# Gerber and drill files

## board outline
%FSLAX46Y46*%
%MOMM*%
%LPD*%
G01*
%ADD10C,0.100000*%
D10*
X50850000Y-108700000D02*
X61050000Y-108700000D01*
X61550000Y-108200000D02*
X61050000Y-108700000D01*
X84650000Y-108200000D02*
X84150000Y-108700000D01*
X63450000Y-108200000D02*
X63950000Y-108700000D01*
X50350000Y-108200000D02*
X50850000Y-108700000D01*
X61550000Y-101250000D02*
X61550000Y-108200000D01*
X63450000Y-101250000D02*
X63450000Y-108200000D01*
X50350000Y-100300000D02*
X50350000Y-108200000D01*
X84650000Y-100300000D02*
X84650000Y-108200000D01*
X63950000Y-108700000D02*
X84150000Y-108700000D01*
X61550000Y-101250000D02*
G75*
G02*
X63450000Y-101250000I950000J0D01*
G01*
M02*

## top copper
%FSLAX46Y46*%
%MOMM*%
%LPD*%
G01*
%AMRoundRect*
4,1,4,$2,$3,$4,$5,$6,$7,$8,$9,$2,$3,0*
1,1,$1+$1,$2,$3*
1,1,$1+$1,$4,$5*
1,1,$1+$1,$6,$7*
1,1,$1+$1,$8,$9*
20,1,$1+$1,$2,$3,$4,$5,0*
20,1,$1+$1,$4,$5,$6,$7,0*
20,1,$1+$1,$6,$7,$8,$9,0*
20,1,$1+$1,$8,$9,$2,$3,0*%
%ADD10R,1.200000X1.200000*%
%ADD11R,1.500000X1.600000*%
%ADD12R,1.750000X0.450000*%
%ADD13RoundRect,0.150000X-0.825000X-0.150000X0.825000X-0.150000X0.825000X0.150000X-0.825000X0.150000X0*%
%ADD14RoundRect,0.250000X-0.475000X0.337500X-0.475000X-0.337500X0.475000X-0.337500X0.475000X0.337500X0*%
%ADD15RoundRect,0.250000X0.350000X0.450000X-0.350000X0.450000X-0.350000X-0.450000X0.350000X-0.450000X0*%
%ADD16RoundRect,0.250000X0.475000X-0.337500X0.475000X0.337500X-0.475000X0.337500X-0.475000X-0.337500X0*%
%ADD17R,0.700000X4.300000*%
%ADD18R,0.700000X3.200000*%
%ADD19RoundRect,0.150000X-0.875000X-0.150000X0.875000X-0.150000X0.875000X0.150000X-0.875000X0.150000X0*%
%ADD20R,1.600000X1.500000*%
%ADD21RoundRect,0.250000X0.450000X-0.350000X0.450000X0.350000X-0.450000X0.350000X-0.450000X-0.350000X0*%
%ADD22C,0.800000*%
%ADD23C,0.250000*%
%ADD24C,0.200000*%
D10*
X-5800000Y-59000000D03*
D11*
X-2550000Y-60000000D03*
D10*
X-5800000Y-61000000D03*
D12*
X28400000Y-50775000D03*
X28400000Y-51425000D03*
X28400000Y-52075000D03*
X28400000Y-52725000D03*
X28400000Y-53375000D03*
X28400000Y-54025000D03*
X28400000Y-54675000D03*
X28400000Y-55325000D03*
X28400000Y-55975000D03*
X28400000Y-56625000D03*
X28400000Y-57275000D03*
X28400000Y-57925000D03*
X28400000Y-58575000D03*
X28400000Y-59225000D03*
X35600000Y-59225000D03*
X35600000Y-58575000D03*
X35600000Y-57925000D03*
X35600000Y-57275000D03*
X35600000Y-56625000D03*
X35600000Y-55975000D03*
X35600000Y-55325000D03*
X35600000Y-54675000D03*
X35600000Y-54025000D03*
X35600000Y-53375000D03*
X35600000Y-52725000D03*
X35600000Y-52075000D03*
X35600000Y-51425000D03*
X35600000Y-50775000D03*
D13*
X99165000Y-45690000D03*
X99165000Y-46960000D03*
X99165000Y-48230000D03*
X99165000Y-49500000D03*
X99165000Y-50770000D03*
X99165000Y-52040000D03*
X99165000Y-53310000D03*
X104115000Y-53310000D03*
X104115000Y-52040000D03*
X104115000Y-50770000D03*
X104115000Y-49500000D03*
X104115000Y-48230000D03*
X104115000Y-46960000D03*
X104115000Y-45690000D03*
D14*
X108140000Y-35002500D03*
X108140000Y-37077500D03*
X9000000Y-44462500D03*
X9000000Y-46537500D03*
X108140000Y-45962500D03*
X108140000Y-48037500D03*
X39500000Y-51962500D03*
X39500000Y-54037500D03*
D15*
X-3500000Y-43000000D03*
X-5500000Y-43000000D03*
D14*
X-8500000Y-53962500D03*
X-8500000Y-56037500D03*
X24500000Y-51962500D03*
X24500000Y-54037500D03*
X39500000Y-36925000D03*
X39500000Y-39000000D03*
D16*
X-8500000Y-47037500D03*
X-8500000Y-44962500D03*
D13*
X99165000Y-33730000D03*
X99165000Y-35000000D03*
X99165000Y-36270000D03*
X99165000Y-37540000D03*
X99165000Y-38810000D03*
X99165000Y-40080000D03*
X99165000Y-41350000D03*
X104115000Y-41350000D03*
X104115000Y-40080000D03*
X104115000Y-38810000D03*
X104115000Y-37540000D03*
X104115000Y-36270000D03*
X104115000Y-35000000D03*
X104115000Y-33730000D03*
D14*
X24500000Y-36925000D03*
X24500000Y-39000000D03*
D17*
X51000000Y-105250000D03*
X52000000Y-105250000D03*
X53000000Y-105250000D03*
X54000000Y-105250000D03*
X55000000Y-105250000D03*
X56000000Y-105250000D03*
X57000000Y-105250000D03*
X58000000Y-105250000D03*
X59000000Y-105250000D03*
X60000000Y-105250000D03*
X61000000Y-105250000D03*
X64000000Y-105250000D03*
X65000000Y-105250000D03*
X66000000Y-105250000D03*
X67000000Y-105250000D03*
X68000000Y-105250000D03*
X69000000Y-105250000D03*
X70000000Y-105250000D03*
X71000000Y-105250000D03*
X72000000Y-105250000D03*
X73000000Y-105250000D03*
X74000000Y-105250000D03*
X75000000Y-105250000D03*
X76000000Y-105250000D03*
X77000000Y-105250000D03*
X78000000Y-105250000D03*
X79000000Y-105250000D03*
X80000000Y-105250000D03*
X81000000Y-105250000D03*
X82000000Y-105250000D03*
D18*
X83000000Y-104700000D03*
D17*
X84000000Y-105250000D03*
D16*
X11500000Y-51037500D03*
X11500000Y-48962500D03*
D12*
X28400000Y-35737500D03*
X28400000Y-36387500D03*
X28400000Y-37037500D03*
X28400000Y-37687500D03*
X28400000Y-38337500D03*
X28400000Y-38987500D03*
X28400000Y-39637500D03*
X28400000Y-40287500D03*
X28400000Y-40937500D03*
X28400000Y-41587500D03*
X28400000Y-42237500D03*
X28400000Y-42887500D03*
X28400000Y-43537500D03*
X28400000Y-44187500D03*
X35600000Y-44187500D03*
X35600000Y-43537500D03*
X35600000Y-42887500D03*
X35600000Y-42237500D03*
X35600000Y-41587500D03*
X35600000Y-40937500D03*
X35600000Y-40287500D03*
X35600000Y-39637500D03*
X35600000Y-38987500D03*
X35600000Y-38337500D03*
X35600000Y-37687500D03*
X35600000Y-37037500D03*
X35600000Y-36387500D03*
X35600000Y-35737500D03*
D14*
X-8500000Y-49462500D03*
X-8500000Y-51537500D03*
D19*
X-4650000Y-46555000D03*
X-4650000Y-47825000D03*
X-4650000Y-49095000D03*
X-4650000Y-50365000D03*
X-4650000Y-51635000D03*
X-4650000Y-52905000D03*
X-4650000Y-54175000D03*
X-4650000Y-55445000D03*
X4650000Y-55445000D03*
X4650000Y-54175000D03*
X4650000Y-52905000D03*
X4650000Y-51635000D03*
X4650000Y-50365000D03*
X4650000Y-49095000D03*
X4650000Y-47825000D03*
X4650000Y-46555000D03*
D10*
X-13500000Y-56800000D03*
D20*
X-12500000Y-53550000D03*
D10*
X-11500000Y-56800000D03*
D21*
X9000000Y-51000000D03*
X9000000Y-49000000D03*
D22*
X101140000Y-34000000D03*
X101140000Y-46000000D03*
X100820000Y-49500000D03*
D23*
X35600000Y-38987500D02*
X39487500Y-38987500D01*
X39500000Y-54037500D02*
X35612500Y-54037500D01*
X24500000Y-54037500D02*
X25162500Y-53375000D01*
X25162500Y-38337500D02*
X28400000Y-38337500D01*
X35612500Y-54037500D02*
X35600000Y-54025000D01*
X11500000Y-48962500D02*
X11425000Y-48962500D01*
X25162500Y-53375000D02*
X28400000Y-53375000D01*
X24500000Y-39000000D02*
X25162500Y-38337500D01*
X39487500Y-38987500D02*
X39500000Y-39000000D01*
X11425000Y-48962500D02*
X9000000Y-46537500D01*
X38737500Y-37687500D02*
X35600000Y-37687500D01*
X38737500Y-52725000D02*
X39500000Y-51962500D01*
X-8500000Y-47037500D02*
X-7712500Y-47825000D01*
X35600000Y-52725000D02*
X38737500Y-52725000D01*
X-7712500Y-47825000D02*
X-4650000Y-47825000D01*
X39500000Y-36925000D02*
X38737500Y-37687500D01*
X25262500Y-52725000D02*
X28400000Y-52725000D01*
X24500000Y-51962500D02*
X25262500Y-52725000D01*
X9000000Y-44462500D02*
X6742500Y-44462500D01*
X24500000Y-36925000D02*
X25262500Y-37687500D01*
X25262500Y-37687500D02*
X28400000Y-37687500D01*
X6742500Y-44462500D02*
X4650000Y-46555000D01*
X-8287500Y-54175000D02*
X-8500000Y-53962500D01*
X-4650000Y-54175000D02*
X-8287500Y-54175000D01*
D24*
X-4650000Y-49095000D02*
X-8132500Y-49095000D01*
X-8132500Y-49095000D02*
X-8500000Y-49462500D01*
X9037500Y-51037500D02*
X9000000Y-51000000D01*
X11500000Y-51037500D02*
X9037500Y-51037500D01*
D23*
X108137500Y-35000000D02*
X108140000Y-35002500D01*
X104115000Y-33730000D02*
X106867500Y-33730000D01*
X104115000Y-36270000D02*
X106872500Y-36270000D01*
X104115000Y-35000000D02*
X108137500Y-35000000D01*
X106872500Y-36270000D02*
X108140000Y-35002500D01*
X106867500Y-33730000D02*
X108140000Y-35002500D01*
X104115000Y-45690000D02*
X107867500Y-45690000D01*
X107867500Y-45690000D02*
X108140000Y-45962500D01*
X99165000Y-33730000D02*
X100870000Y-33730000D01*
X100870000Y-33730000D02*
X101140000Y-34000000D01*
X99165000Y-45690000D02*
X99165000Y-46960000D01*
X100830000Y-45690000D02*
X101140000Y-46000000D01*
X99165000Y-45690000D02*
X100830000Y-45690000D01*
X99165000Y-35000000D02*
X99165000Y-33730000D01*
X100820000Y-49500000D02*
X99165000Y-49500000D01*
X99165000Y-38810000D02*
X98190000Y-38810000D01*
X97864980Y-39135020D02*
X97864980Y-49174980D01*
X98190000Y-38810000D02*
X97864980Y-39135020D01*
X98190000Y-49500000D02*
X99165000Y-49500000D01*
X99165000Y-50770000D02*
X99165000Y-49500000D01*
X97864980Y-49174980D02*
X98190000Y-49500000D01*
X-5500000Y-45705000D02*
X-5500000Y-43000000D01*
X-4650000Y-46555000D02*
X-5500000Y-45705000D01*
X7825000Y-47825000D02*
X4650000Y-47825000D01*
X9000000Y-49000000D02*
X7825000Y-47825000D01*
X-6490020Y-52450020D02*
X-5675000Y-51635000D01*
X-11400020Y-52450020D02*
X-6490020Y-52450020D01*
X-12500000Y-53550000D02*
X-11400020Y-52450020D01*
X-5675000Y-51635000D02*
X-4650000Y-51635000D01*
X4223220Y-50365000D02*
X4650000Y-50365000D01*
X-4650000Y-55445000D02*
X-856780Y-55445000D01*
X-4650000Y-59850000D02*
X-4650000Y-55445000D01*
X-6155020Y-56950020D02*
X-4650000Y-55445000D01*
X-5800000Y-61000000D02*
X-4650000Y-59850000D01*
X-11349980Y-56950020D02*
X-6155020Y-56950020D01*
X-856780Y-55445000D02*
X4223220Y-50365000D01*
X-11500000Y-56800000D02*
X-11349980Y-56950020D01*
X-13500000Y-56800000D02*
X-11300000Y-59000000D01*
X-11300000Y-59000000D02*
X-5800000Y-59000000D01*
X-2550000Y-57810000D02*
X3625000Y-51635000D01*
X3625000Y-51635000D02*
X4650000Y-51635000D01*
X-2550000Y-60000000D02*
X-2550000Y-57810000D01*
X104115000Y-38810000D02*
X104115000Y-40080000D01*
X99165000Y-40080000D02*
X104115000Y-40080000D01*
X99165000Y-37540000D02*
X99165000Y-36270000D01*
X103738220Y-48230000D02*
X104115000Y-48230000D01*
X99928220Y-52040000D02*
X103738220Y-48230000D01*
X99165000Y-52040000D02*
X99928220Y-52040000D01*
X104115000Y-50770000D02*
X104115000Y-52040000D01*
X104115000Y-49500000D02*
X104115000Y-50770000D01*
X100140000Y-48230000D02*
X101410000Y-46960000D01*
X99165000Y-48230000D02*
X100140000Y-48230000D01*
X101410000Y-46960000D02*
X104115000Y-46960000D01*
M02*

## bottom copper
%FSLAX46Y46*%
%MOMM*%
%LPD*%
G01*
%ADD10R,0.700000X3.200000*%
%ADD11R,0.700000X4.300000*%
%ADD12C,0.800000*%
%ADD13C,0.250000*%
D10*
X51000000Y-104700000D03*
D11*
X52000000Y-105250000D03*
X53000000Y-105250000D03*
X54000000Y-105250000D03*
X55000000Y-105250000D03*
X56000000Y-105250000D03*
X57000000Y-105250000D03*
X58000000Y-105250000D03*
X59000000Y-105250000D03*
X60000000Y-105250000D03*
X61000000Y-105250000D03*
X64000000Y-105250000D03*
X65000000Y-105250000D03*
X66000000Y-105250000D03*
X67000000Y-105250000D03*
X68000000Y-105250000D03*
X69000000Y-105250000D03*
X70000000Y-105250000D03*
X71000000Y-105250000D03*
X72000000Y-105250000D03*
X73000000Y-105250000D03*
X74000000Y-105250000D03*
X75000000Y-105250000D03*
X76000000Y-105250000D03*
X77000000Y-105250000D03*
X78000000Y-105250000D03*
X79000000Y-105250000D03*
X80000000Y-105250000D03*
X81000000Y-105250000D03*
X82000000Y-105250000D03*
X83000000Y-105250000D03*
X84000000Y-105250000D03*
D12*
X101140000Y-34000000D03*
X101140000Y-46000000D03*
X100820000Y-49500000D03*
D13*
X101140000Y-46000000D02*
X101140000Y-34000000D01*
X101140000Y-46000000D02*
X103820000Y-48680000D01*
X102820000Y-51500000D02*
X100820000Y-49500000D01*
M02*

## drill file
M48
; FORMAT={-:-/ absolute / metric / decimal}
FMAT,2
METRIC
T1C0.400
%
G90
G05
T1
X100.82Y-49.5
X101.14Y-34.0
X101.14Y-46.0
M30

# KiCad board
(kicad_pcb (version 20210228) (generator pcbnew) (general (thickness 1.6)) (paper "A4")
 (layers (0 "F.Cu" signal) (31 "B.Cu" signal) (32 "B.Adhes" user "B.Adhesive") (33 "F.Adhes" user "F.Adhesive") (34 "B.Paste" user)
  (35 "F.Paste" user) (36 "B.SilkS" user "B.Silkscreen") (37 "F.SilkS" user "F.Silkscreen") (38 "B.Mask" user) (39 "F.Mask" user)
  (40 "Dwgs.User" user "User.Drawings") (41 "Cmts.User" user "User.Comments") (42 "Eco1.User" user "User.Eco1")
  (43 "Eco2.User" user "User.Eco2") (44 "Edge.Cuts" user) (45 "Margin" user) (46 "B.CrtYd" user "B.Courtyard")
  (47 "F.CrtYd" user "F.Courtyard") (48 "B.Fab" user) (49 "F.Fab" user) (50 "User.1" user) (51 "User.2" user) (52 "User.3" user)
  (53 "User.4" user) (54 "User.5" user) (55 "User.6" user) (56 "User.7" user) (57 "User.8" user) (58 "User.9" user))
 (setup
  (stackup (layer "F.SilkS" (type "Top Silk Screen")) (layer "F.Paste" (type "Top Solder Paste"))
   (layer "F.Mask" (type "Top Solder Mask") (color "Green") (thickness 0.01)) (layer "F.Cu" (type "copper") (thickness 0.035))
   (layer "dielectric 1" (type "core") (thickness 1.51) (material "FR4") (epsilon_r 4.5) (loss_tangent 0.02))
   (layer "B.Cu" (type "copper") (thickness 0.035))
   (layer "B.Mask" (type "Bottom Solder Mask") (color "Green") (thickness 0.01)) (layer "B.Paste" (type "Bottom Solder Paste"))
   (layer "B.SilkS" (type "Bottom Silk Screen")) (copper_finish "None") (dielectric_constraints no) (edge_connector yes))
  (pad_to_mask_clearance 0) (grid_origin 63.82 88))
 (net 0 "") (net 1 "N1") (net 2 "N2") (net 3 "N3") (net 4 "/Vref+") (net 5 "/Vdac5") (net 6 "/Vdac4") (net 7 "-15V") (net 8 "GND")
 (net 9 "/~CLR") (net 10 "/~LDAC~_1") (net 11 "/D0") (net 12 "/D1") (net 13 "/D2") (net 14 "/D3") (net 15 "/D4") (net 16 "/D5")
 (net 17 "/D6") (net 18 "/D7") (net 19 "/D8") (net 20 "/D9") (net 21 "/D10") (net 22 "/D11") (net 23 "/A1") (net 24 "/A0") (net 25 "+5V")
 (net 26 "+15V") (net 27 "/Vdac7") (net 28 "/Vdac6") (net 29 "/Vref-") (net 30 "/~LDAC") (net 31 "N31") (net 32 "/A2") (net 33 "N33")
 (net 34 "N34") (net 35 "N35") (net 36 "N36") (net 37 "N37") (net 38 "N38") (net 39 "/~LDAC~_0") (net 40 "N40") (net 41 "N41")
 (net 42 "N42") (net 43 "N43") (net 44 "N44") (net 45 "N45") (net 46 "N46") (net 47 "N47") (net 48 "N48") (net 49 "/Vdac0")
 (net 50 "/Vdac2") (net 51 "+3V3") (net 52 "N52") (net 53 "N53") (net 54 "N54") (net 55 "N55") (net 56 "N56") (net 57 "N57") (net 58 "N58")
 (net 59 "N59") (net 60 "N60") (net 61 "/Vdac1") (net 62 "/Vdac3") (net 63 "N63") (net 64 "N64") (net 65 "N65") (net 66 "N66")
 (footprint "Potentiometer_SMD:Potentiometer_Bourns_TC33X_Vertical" (layer "F.Cu") (at -4 60)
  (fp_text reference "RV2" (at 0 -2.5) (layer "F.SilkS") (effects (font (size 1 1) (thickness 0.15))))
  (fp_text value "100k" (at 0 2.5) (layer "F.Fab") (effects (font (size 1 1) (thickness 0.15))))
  (pad "1" smd rect (at -1.8 -1) (locked) (size 1.2 1.2) (layers "F.Cu" "F.Paste" "F.Mask") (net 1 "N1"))
  (pad "2" smd rect (at 1.45 0) (locked) (size 1.5 1.6) (layers "F.Cu" "F.Paste" "F.Mask") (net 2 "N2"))
  (pad "3" smd rect (at -1.8 1) (locked) (size 1.2 1.2) (layers "F.Cu" "F.Paste" "F.Mask") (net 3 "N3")))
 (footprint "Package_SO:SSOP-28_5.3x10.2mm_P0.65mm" (layer "F.Cu") (at 32 55)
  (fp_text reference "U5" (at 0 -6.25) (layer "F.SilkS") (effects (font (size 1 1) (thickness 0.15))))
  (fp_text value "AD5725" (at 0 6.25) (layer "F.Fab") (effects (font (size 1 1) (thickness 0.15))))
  (pad "1" smd rect (at -3.6 -4.225) (locked) (size 1.75 0.45) (layers "F.Cu" "F.Paste" "F.Mask") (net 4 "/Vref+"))
  (pad "2" smd rect (at -3.6 -3.575) (locked) (size 1.75 0.45) (layers "F.Cu" "F.Paste" "F.Mask") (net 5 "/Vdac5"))
  (pad "3" smd rect (at -3.6 -2.925) (locked) (size 1.75 0.45) (layers "F.Cu" "F.Paste" "F.Mask") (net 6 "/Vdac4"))
  (pad "4" smd rect (at -3.6 -2.275) (locked) (size 1.75 0.45) (layers "F.Cu" "F.Paste" "F.Mask") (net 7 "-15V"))
  (pad "5" smd rect (at -3.6 -1.625) (locked) (size 1.75 0.45) (layers "F.Cu" "F.Paste" "F.Mask") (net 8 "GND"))
  (pad "6" smd rect (at -3.6 -0.975) (locked) (size 1.75 0.45) (layers "F.Cu" "F.Paste" "F.Mask") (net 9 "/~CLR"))
  (pad "7" smd rect (at -3.6 -0.325) (locked) (size 1.75 0.45) (layers "F.Cu" "F.Paste" "F.Mask") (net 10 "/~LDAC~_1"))
  (pad "8" smd rect (at -3.6 0.325) (locked) (size 1.75 0.45) (layers "F.Cu" "F.Paste" "F.Mask") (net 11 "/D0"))
  (pad "9" smd rect (at -3.6 0.975) (locked) (size 1.75 0.45) (layers "F.Cu" "F.Paste" "F.Mask") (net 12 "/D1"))
  (pad "10" smd rect (at -3.6 1.625) (locked) (size 1.75 0.45) (layers "F.Cu" "F.Paste" "F.Mask") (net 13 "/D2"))
  (pad "11" smd rect (at -3.6 2.275) (locked) (size 1.75 0.45) (layers "F.Cu" "F.Paste" "F.Mask") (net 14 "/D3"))
  (pad "12" smd rect (at -3.6 2.925) (locked) (size 1.75 0.45) (layers "F.Cu" "F.Paste" "F.Mask") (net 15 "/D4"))
  (pad "13" smd rect (at -3.6 3.575) (locked) (size 1.75 0.45) (layers "F.Cu" "F.Paste" "F.Mask") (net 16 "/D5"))
  (pad "14" smd rect (at -3.6 4.225) (locked) (size 1.75 0.45) (layers "F.Cu" "F.Paste" "F.Mask") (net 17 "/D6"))
  (pad "15" smd rect (at 3.6 4.225) (locked) (size 1.75 0.45) (layers "F.Cu" "F.Paste" "F.Mask") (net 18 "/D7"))
  (pad "16" smd rect (at 3.6 3.575) (locked) (size 1.75 0.45) (layers "F.Cu" "F.Paste" "F.Mask") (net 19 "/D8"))
  (pad "17" smd rect (at 3.6 2.925) (locked) (size 1.75 0.45) (layers "F.Cu" "F.Paste" "F.Mask") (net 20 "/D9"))
  (pad "18" smd rect (at 3.6 2.275) (locked) (size 1.75 0.45) (layers "F.Cu" "F.Paste" "F.Mask") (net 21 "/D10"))
  (pad "19" smd rect (at 3.6 1.625) (locked) (size 1.75 0.45) (layers "F.Cu" "F.Paste" "F.Mask") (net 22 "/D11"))
  (pad "20" smd rect (at 3.6 0.975) (locked) (size 1.75 0.45) (layers "F.Cu" "F.Paste" "F.Mask") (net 8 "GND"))
  (pad "21" smd rect (at 3.6 0.325) (locked) (size 1.75 0.45) (layers "F.Cu" "F.Paste" "F.Mask") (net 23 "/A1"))
  (pad "22" smd rect (at 3.6 -0.325) (locked) (size 1.75 0.45) (layers "F.Cu" "F.Paste" "F.Mask") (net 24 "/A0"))
  (pad "23" smd rect (at 3.6 -0.975) (locked) (size 1.75 0.45) (layers "F.Cu" "F.Paste" "F.Mask") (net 8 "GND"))
  (pad "24" smd rect (at 3.6 -1.625) (locked) (size 1.75 0.45) (layers "F.Cu" "F.Paste" "F.Mask") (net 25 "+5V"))
  (pad "25" smd rect (at 3.6 -2.275) (locked) (size 1.75 0.45) (layers "F.Cu" "F.Paste" "F.Mask") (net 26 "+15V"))
  (pad "26" smd rect (at 3.6 -2.925) (locked) (size 1.75 0.45) (layers "F.Cu" "F.Paste" "F.Mask") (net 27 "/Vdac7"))
  (pad "27" smd rect (at 3.6 -3.575) (locked) (size 1.75 0.45) (layers "F.Cu" "F.Paste" "F.Mask") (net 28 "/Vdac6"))
  (pad "28" smd rect (at 3.6 -4.225) (locked) (size 1.75 0.45) (layers "F.Cu" "F.Paste" "F.Mask") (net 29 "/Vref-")))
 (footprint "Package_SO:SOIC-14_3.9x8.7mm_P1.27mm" (layer "F.Cu") (at 101.64 49.5)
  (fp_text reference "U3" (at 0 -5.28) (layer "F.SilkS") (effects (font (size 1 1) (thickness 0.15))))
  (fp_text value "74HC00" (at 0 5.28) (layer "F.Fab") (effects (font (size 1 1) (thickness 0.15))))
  (pad "1" smd roundrect (at -2.475 -3.81) (locked) (size 1.95 0.6) (layers "F.Cu" "F.Paste" "F.Mask") (roundrect_rratio 0.25)
   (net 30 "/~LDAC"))
  (pad "2" smd roundrect (at -2.475 -2.54) (locked) (size 1.95 0.6) (layers "F.Cu" "F.Paste" "F.Mask") (roundrect_rratio 0.25)
   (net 30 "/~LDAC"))
  (pad "3" smd roundrect (at -2.475 -1.27) (locked) (size 1.95 0.6) (layers "F.Cu" "F.Paste" "F.Mask") (roundrect_rratio 0.25)
   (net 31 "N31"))
  (pad "4" smd roundrect (at -2.475 0) (locked) (size 1.95 0.6) (layers "F.Cu" "F.Paste" "F.Mask") (roundrect_rratio 0.25) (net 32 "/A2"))
  (pad "5" smd roundrect (at -2.475 1.27) (locked) (size 1.95 0.6) (layers "F.Cu" "F.Paste" "F.Mask") (roundrect_rratio 0.25) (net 32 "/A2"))
  (pad "6" smd roundrect (at -2.475 2.54) (locked) (size 1.95 0.6) (layers "F.Cu" "F.Paste" "F.Mask") (roundrect_rratio 0.25) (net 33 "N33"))
  (pad "7" smd roundrect (at -2.475 3.81) (locked) (size 1.95 0.6) (layers "F.Cu" "F.Paste" "F.Mask") (roundrect_rratio 0.25) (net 8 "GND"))
  (pad "8" smd roundrect (at 2.475 3.81) (locked) (size 1.95 0.6) (layers "F.Cu" "F.Paste" "F.Mask") (roundrect_rratio 0.25)
   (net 10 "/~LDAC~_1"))
  (pad "9" smd roundrect (at 2.475 2.54) (locked) (size 1.95 0.6) (layers "F.Cu" "F.Paste" "F.Mask") (roundrect_rratio 0.25) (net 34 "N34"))
  (pad "10" smd roundrect (at 2.475 1.27) (locked) (size 1.95 0.6) (layers "F.Cu" "F.Paste" "F.Mask") (roundrect_rratio 0.25) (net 34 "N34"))
  (pad "11" smd roundrect (at 2.475 0) (locked) (size 1.95 0.6) (layers "F.Cu" "F.Paste" "F.Mask") (roundrect_rratio 0.25) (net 34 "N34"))
  (pad "12" smd roundrect (at 2.475 -1.27) (locked) (size 1.95 0.6) (layers "F.Cu" "F.Paste" "F.Mask") (roundrect_rratio 0.25)
   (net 33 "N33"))
  (pad "13" smd roundrect (at 2.475 -2.54) (locked) (size 1.95 0.6) (layers "F.Cu" "F.Paste" "F.Mask") (roundrect_rratio 0.25)
   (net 31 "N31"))
  (pad "14" smd roundrect (at 2.475 -3.81) (locked) (size 1.95 0.6) (layers "F.Cu" "F.Paste" "F.Mask") (roundrect_rratio 0.25)
   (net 25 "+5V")))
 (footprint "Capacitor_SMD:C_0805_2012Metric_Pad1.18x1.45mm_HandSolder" (layer "F.Cu") (at 108.14 36.04 -90)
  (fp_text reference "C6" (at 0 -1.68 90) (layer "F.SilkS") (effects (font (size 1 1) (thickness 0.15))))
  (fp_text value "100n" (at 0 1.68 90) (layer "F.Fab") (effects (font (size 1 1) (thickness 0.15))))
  (pad "1" smd roundrect (at -1.0375 0 270) (locked) (size 1.175 1.45) (layers "F.Cu" "F.Paste" "F.Mask") (roundrect_rratio 0.212766)
   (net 25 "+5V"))
  (pad "2" smd roundrect (at 1.0375 0 270) (locked) (size 1.175 1.45) (layers "F.Cu" "F.Paste" "F.Mask") (roundrect_rratio 0.212766)
   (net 8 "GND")))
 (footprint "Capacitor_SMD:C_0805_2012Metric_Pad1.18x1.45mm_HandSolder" (layer "F.Cu") (at 9 45.5 -90)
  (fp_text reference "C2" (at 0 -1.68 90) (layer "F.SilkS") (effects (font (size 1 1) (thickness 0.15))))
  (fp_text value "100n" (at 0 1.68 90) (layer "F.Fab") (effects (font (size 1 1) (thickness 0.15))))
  (pad "1" smd roundrect (at -1.0375 0 270) (locked) (size 1.175 1.45) (layers "F.Cu" "F.Paste" "F.Mask") (roundrect_rratio 0.212766)
   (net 7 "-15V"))
  (pad "2" smd roundrect (at 1.0375 0 270) (locked) (size 1.175 1.45) (layers "F.Cu" "F.Paste" "F.Mask") (roundrect_rratio 0.212766)
   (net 8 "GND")))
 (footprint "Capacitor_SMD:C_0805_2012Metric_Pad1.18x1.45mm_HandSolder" (layer "F.Cu") (at 108.14 47 -90)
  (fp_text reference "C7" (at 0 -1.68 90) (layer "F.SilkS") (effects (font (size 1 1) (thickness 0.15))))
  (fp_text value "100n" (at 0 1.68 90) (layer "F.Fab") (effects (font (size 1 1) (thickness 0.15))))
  (pad "1" smd roundrect (at -1.0375 0 270) (locked) (size 1.175 1.45) (layers "F.Cu" "F.Paste" "F.Mask") (roundrect_rratio 0.212766)
   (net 25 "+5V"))
  (pad "2" smd roundrect (at 1.0375 0 270) (locked) (size 1.175 1.45) (layers "F.Cu" "F.Paste" "F.Mask") (roundrect_rratio 0.212766)
   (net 8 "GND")))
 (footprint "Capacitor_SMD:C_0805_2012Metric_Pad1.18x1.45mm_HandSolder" (layer "F.Cu") (at 39.5 53 -90)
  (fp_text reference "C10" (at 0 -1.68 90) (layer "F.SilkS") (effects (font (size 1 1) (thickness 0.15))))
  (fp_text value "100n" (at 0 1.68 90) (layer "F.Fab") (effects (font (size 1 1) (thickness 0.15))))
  (pad "1" smd roundrect (at -1.0375 0 270) (locked) (size 1.175 1.45) (layers "F.Cu" "F.Paste" "F.Mask") (roundrect_rratio 0.212766)
   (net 26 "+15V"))
  (pad "2" smd roundrect (at 1.0375 0 270) (locked) (size 1.175 1.45) (layers "F.Cu" "F.Paste" "F.Mask") (roundrect_rratio 0.212766)
   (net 8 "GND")))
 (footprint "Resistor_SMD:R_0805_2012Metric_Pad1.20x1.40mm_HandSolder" (layer "F.Cu") (at -4.5 43 180)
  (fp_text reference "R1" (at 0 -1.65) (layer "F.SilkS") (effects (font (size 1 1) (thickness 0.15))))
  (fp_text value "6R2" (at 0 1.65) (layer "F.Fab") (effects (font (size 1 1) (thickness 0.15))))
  (pad "1" smd roundrect (at -1 0 180) (locked) (size 1.2 1.4) (layers "F.Cu" "F.Paste" "F.Mask") (roundrect_rratio 0.208333)
   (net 4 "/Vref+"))
  (pad "2" smd roundrect (at 1 0 180) (locked) (size 1.2 1.4) (layers "F.Cu" "F.Paste" "F.Mask") (roundrect_rratio 0.208333) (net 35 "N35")))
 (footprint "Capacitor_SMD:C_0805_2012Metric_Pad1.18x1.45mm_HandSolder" (layer "F.Cu") (at -8.5 55 -90)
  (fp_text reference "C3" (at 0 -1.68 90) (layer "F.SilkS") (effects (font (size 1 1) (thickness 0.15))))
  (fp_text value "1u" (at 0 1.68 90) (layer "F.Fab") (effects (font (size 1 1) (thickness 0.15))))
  (pad "1" smd roundrect (at -1.0375 0 270) (locked) (size 1.175 1.45) (layers "F.Cu" "F.Paste" "F.Mask") (roundrect_rratio 0.212766)
   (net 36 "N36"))
  (pad "2" smd roundrect (at 1.0375 0 270) (locked) (size 1.175 1.45) (layers "F.Cu" "F.Paste" "F.Mask") (roundrect_rratio 0.212766)
   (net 8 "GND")))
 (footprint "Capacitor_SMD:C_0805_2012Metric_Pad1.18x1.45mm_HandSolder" (layer "F.Cu") (at 24.5 53 -90)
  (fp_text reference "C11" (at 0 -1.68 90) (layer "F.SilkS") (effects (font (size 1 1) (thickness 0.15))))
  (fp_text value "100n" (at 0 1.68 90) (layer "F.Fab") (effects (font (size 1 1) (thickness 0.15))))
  (pad "1" smd roundrect (at -1.0375 0 270) (locked) (size 1.175 1.45) (layers "F.Cu" "F.Paste" "F.Mask") (roundrect_rratio 0.212766)
   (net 7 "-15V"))
  (pad "2" smd roundrect (at 1.0375 0 270) (locked) (size 1.175 1.45) (layers "F.Cu" "F.Paste" "F.Mask") (roundrect_rratio 0.212766)
   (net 8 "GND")))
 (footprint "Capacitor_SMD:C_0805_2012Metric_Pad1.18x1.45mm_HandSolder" (layer "F.Cu") (at 39.5 37.9625 -90)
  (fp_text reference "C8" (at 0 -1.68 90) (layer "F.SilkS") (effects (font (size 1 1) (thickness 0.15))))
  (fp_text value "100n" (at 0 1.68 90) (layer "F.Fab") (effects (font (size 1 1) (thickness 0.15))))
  (pad "1" smd roundrect (at -1.0375 0 270) (locked) (size 1.175 1.45) (layers "F.Cu" "F.Paste" "F.Mask") (roundrect_rratio 0.212766)
   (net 26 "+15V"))
  (pad "2" smd roundrect (at 1.0375 0 270) (locked) (size 1.175 1.45) (layers "F.Cu" "F.Paste" "F.Mask") (roundrect_rratio 0.212766)
   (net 8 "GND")))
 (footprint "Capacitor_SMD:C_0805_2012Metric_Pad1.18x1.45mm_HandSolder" (layer "F.Cu") (at -8.5 46 90)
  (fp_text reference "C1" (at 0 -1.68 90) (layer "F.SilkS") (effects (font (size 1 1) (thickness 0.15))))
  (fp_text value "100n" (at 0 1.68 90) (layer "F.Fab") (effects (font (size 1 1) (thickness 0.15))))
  (pad "1" smd roundrect (at -1.0375 0 90) (locked) (size 1.175 1.45) (layers "F.Cu" "F.Paste" "F.Mask") (roundrect_rratio 0.212766)
   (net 26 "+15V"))
  (pad "2" smd roundrect (at 1.0375 0 90) (locked) (size 1.175 1.45) (layers "F.Cu" "F.Paste" "F.Mask") (roundrect_rratio 0.212766)
   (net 8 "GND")))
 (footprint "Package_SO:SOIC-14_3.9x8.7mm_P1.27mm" (layer "F.Cu") (at 101.64 37.54)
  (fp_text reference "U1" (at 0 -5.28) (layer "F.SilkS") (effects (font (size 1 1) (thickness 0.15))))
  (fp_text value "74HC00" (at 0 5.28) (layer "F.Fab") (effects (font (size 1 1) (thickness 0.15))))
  (pad "1" smd roundrect (at -2.475 -3.81) (locked) (size 1.95 0.6) (layers "F.Cu" "F.Paste" "F.Mask") (roundrect_rratio 0.25)
   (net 30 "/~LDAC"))
  (pad "2" smd roundrect (at -2.475 -2.54) (locked) (size 1.95 0.6) (layers "F.Cu" "F.Paste" "F.Mask") (roundrect_rratio 0.25)
   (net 30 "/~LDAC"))
  (pad "3" smd roundrect (at -2.475 -1.27) (locked) (size 1.95 0.6) (layers "F.Cu" "F.Paste" "F.Mask") (roundrect_rratio 0.25)
   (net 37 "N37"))
  (pad "4" smd roundrect (at -2.475 0) (locked) (size 1.95 0.6) (layers "F.Cu" "F.Paste" "F.Mask") (roundrect_rratio 0.25) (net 37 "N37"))
  (pad "5" smd roundrect (at -2.475 1.27) (locked) (size 1.95 0.6) (layers "F.Cu" "F.Paste" "F.Mask") (roundrect_rratio 0.25) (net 32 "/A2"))
  (pad "6" smd roundrect (at -2.475 2.54) (locked) (size 1.95 0.6) (layers "F.Cu" "F.Paste" "F.Mask") (roundrect_rratio 0.25) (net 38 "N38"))
  (pad "7" smd roundrect (at -2.475 3.81) (locked) (size 1.95 0.6) (layers "F.Cu" "F.Paste" "F.Mask") (roundrect_rratio 0.25) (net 8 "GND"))
  (pad "8" smd roundrect (at 2.475 3.81) (locked) (size 1.95 0.6) (layers "F.Cu" "F.Paste" "F.Mask") (roundrect_rratio 0.25)
   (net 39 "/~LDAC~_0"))
  (pad "9" smd roundrect (at 2.475 2.54) (locked) (size 1.95 0.6) (layers "F.Cu" "F.Paste" "F.Mask") (roundrect_rratio 0.25) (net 38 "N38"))
  (pad "10" smd roundrect (at 2.475 1.27) (locked) (size 1.95 0.6) (layers "F.Cu" "F.Paste" "F.Mask") (roundrect_rratio 0.25) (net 38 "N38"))
  (pad "11" smd roundrect (at 2.475 0) (locked) (size 1.95 0.6) (layers "F.Cu" "F.Paste" "F.Mask") (roundrect_rratio 0.25) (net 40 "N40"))
  (pad "12" smd roundrect (at 2.475 -1.27) (locked) (size 1.95 0.6) (layers "F.Cu" "F.Paste" "F.Mask") (roundrect_rratio 0.25)
   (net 25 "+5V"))
  (pad "13" smd roundrect (at 2.475 -2.54) (locked) (size 1.95 0.6) (layers "F.Cu" "F.Paste" "F.Mask") (roundrect_rratio 0.25)
   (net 25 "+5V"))
  (pad "14" smd roundrect (at 2.475 -3.81) (locked) (size 1.95 0.6) (layers "F.Cu" "F.Paste" "F.Mask") (roundrect_rratio 0.25)
   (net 25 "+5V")))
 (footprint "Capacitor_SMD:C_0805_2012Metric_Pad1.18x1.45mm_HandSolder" (layer "F.Cu") (at 24.5 37.9625 -90)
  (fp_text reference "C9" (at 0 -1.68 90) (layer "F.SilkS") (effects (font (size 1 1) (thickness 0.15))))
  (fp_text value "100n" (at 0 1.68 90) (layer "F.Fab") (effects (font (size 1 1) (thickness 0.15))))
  (pad "1" smd roundrect (at -1.0375 0 270) (locked) (size 1.175 1.45) (layers "F.Cu" "F.Paste" "F.Mask") (roundrect_rratio 0.212766)
   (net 7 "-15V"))
  (pad "2" smd roundrect (at 1.0375 0 270) (locked) (size 1.175 1.45) (layers "F.Cu" "F.Paste" "F.Mask") (roundrect_rratio 0.212766)
   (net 8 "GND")))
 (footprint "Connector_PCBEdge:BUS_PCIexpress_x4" (layer "F.Cu") (at 51 105.25)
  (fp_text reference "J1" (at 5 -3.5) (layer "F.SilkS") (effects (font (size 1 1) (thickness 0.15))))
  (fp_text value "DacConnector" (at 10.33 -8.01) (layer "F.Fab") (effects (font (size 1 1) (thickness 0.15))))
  (fp_line (start -0.15 3.45) (end 10.05 3.45) (layer "Edge.Cuts") (width 0.1))
  (fp_line (start 10.55 2.95) (end 10.05 3.45) (layer "Edge.Cuts") (width 0.1))
  (fp_line (start 33.65 2.95) (end 33.15 3.45) (layer "Edge.Cuts") (width 0.1))
  (fp_line (start 12.45 2.95) (end 12.95 3.45) (layer "Edge.Cuts") (width 0.1))
  (fp_line (start -0.65 2.95) (end -0.15 3.45) (layer "Edge.Cuts") (width 0.1))
  (fp_line (start 10.55 -4) (end 10.55 2.95) (layer "Edge.Cuts") (width 0.1))
  (fp_line (start 12.45 -4) (end 12.45 2.95) (layer "Edge.Cuts") (width 0.1))
  (fp_line (start -0.65 -4.95) (end -0.65 2.95) (layer "Edge.Cuts") (width 0.1))
  (fp_line (start 33.65 -4.95) (end 33.65 2.95) (layer "Edge.Cuts") (width 0.1))
  (fp_line (start 12.95 3.45) (end 33.15 3.45) (layer "Edge.Cuts") (width 0.1))
  (fp_arc (start 11.5 -4) (end 12.45 -4) (angle -180) (layer "Edge.Cuts") (width 0.1))
  (pad "A1" connect rect (at 0 -0.55) (locked) (size 0.7 3.2) (layers "B.Cu" "B.Mask") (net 26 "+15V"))
  (pad "A2" connect rect (at 1 0) (locked) (size 0.7 4.3) (layers "B.Cu" "B.Mask") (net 8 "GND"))
  (pad "A3" connect rect (at 2 0) (locked) (size 0.7 4.3) (layers "B.Cu" "B.Mask") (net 7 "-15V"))
  (pad "A4" connect rect (at 3 0) (locked) (size 0.7 4.3) (layers "B.Cu" "B.Mask") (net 8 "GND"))
  (pad "A5" connect rect (at 4 0) (locked) (size 0.7 4.3) (layers "B.Cu" "B.Mask") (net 25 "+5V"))
  (pad "A6" connect rect (at 5 0) (locked) (size 0.7 4.3) (layers "B.Cu" "B.Mask") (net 11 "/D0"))
  (pad "A7" connect rect (at 6 0) (locked) (size 0.7 4.3) (layers "B.Cu" "B.Mask") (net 13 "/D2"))
  (pad "A8" connect rect (at 7 0) (locked) (size 0.7 4.3) (layers "B.Cu" "B.Mask") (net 15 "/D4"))
  (pad "A9" connect rect (at 8 0) (locked) (size 0.7 4.3) (layers "B.Cu" "B.Mask") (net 17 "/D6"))
  (pad "A10" connect rect (at 9 0) (locked) (size 0.7 4.3) (layers "B.Cu" "B.Mask") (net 19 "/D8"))
  (pad "A11" connect rect (at 10 0) (locked) (size 0.7 4.3) (layers "B.Cu" "B.Mask") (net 21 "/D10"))
  (pad "A12" connect rect (at 13 0) (locked) (size 0.7 4.3) (layers "B.Cu" "B.Mask") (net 24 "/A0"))
  (pad "A13" connect rect (at 14 0) (locked) (size 0.7 4.3) (layers "B.Cu" "B.Mask") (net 32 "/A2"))
  (pad "A14" connect rect (at 15 0) (locked) (size 0.7 4.3) (layers "B.Cu" "B.Mask") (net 30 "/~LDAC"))
  (pad "A15" connect rect (at 16 0) (locked) (size 0.7 4.3) (layers "B.Cu" "B.Mask") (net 8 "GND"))
  (pad "A16" connect rect (at 17 0) (locked) (size 0.7 4.3) (layers "B.Cu" "B.Mask") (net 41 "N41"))
  (pad "A17" connect rect (at 18 0) (locked) (size 0.7 4.3) (layers "B.Cu" "B.Mask") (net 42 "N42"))
  (pad "A18" connect rect (at 19 0) (locked) (size 0.7 4.3) (layers "B.Cu" "B.Mask") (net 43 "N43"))
  (pad "A19" connect rect (at 20 0) (locked) (size 0.7 4.3) (layers "B.Cu" "B.Mask") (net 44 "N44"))
  (pad "A20" connect rect (at 21 0) (locked) (size 0.7 4.3) (layers "B.Cu" "B.Mask") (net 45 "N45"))
  (pad "A21" connect rect (at 22 0) (locked) (size 0.7 4.3) (layers "B.Cu" "B.Mask") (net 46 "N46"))
  (pad "A22" connect rect (at 23 0) (locked) (size 0.7 4.3) (layers "B.Cu" "B.Mask") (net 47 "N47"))
  (pad "A23" connect rect (at 24 0) (locked) (size 0.7 4.3) (layers "B.Cu" "B.Mask") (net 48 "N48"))
  (pad "A24" connect rect (at 25 0) (locked) (size 0.7 4.3) (layers "B.Cu" "B.Mask") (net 8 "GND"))
  (pad "A25" connect rect (at 26 0) (locked) (size 0.7 4.3) (layers "B.Cu" "B.Mask") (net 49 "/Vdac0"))
  (pad "A26" connect rect (at 27 0) (locked) (size 0.7 4.3) (layers "B.Cu" "B.Mask") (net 8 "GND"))
  (pad "A27" connect rect (at 28 0) (locked) (size 0.7 4.3) (layers "B.Cu" "B.Mask") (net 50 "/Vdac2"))
  (pad "A28" connect rect (at 29 0) (locked) (size 0.7 4.3) (layers "B.Cu" "B.Mask") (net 8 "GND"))
  (pad "A29" connect rect (at 30 0) (locked) (size 0.7 4.3) (layers "B.Cu" "B.Mask") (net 6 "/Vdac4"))
  (pad "A30" connect rect (at 31 0) (locked) (size 0.7 4.3) (layers "B.Cu" "B.Mask") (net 8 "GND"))
  (pad "A31" connect rect (at 32 0) (locked) (size 0.7 4.3) (layers "B.Cu" "B.Mask") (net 28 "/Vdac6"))
  (pad "A32" connect rect (at 33 0) (locked) (size 0.7 4.3) (layers "B.Cu" "B.Mask") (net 8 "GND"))
  (pad "B1" connect rect (at 0 0) (locked) (size 0.7 4.3) (layers "F.Cu" "F.Mask") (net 26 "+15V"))
  (pad "B2" connect rect (at 1 0) (locked) (size 0.7 4.3) (layers "F.Cu" "F.Mask") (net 8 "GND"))
  (pad "B3" connect rect (at 2 0) (locked) (size 0.7 4.3) (layers "F.Cu" "F.Mask") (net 7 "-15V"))
  (pad "B4" connect rect (at 3 0) (locked) (size 0.7 4.3) (layers "F.Cu" "F.Mask") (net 8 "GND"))
  (pad "B5" connect rect (at 4 0) (locked) (size 0.7 4.3) (layers "F.Cu" "F.Mask") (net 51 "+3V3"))
  (pad "B6" connect rect (at 5 0) (locked) (size 0.7 4.3) (layers "F.Cu" "F.Mask") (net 12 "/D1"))
  (pad "B7" connect rect (at 6 0) (locked) (size 0.7 4.3) (layers "F.Cu" "F.Mask") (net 14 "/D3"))
  (pad "B8" connect rect (at 7 0) (locked) (size 0.7 4.3) (layers "F.Cu" "F.Mask") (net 16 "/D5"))
  (pad "B9" connect rect (at 8 0) (locked) (size 0.7 4.3) (layers "F.Cu" "F.Mask") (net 18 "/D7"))
  (pad "B10" connect rect (at 9 0) (locked) (size 0.7 4.3) (layers "F.Cu" "F.Mask") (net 20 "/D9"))
  (pad "B11" connect rect (at 10 0) (locked) (size 0.7 4.3) (layers "F.Cu" "F.Mask") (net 22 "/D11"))
  (pad "B12" connect rect (at 13 0) (locked) (size 0.7 4.3) (layers "F.Cu" "F.Mask") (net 23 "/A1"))
  (pad "B13" connect rect (at 14 0) (locked) (size 0.7 4.3) (layers "F.Cu" "F.Mask") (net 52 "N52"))
  (pad "B14" connect rect (at 15 0) (locked) (size 0.7 4.3) (layers "F.Cu" "F.Mask") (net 9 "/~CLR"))
  (pad "B15" connect rect (at 16 0) (locked) (size 0.7 4.3) (layers "F.Cu" "F.Mask") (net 8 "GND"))
  (pad "B16" connect rect (at 17 0) (locked) (size 0.7 4.3) (layers "F.Cu" "F.Mask") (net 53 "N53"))
  (pad "B17" connect rect (at 18 0) (locked) (size 0.7 4.3) (layers "F.Cu" "F.Mask") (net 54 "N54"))
  (pad "B18" connect rect (at 19 0) (locked) (size 0.7 4.3) (layers "F.Cu" "F.Mask") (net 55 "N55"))
  (pad "B19" connect rect (at 20 0) (locked) (size 0.7 4.3) (layers "F.Cu" "F.Mask") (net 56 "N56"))
  (pad "B20" connect rect (at 21 0) (locked) (size 0.7 4.3) (layers "F.Cu" "F.Mask") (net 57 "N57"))
  (pad "B21" connect rect (at 22 0) (locked) (size 0.7 4.3) (layers "F.Cu" "F.Mask") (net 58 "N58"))
  (pad "B22" connect rect (at 23 0) (locked) (size 0.7 4.3) (layers "F.Cu" "F.Mask") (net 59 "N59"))
  (pad "B23" connect rect (at 24 0) (locked) (size 0.7 4.3) (layers "F.Cu" "F.Mask") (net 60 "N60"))
  (pad "B24" connect rect (at 25 0) (locked) (size 0.7 4.3) (layers "F.Cu" "F.Mask") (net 8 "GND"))
  (pad "B25" connect rect (at 26 0) (locked) (size 0.7 4.3) (layers "F.Cu" "F.Mask") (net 8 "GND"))
  (pad "B26" connect rect (at 27 0) (locked) (size 0.7 4.3) (layers "F.Cu" "F.Mask") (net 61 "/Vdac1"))
  (pad "B27" connect rect (at 28 0) (locked) (size 0.7 4.3) (layers "F.Cu" "F.Mask") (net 8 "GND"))
  (pad "B28" connect rect (at 29 0) (locked) (size 0.7 4.3) (layers "F.Cu" "F.Mask") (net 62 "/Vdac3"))
  (pad "B29" connect rect (at 30 0) (locked) (size 0.7 4.3) (layers "F.Cu" "F.Mask") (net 8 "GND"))
  (pad "B30" connect rect (at 31 0) (locked) (size 0.7 4.3) (layers "F.Cu" "F.Mask") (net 5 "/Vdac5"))
  (pad "B31" connect rect (at 32 -0.55) (locked) (size 0.7 3.2) (layers "F.Cu" "F.Mask") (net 8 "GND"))
  (pad "B32" connect rect (at 33 0) (locked) (size 0.7 4.3) (layers "F.Cu" "F.Mask") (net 27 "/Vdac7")))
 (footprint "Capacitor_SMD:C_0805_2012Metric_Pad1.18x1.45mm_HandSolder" (layer "F.Cu") (at 11.5 50 90)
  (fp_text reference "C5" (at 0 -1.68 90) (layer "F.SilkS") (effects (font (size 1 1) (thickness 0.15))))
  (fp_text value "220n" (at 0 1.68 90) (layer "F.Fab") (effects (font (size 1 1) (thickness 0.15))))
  (pad "1" smd roundrect (at -1.0375 0 90) (locked) (size 1.175 1.45) (layers "F.Cu" "F.Paste" "F.Mask") (roundrect_rratio 0.212766)
   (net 29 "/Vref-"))
  (pad "2" smd roundrect (at 1.0375 0 90) (locked) (size 1.175 1.45) (layers "F.Cu" "F.Paste" "F.Mask") (roundrect_rratio 0.212766)
   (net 8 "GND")))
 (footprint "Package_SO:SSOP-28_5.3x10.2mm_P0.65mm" (layer "F.Cu") (at 32 39.9625)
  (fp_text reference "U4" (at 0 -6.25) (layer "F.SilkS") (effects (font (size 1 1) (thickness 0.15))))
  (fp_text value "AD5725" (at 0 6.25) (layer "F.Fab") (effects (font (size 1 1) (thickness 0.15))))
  (pad "1" smd rect (at -3.6 -4.225) (locked) (size 1.75 0.45) (layers "F.Cu" "F.Paste" "F.Mask") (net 4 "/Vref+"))
  (pad "2" smd rect (at -3.6 -3.575) (locked) (size 1.75 0.45) (layers "F.Cu" "F.Paste" "F.Mask") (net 61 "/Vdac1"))
  (pad "3" smd rect (at -3.6 -2.925) (locked) (size 1.75 0.45) (layers "F.Cu" "F.Paste" "F.Mask") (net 49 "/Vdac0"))
  (pad "4" smd rect (at -3.6 -2.275) (locked) (size 1.75 0.45) (layers "F.Cu" "F.Paste" "F.Mask") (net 7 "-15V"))
  (pad "5" smd rect (at -3.6 -1.625) (locked) (size 1.75 0.45) (layers "F.Cu" "F.Paste" "F.Mask") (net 8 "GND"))
  (pad "6" smd rect (at -3.6 -0.975) (locked) (size 1.75 0.45) (layers "F.Cu" "F.Paste" "F.Mask") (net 9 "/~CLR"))
  (pad "7" smd rect (at -3.6 -0.325) (locked) (size 1.75 0.45) (layers "F.Cu" "F.Paste" "F.Mask") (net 39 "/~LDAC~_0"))
  (pad "8" smd rect (at -3.6 0.325) (locked) (size 1.75 0.45) (layers "F.Cu" "F.Paste" "F.Mask") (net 11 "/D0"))
  (pad "9" smd rect (at -3.6 0.975) (locked) (size 1.75 0.45) (layers "F.Cu" "F.Paste" "F.Mask") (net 12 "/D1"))
  (pad "10" smd rect (at -3.6 1.625) (locked) (size 1.75 0.45) (layers "F.Cu" "F.Paste" "F.Mask") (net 13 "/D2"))
  (pad "11" smd rect (at -3.6 2.275) (locked) (size 1.75 0.45) (layers "F.Cu" "F.Paste" "F.Mask") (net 14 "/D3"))
  (pad "12" smd rect (at -3.6 2.925) (locked) (size 1.75 0.45) (layers "F.Cu" "F.Paste" "F.Mask") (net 15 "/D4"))
  (pad "13" smd rect (at -3.6 3.575) (locked) (size 1.75 0.45) (layers "F.Cu" "F.Paste" "F.Mask") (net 16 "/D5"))
  (pad "14" smd rect (at -3.6 4.225) (locked) (size 1.75 0.45) (layers "F.Cu" "F.Paste" "F.Mask") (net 17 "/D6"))
  (pad "15" smd rect (at 3.6 4.225) (locked) (size 1.75 0.45) (layers "F.Cu" "F.Paste" "F.Mask") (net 18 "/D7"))
  (pad "16" smd rect (at 3.6 3.575) (locked) (size 1.75 0.45) (layers "F.Cu" "F.Paste" "F.Mask") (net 19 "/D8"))
  (pad "17" smd rect (at 3.6 2.925) (locked) (size 1.75 0.45) (layers "F.Cu" "F.Paste" "F.Mask") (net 20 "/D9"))
  (pad "18" smd rect (at 3.6 2.275) (locked) (size 1.75 0.45) (layers "F.Cu" "F.Paste" "F.Mask") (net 21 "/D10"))
  (pad "19" smd rect (at 3.6 1.625) (locked) (size 1.75 0.45) (layers "F.Cu" "F.Paste" "F.Mask") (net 22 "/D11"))
  (pad "20" smd rect (at 3.6 0.975) (locked) (size 1.75 0.45) (layers "F.Cu" "F.Paste" "F.Mask") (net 8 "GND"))
  (pad "21" smd rect (at 3.6 0.325) (locked) (size 1.75 0.45) (layers "F.Cu" "F.Paste" "F.Mask") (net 23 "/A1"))
  (pad "22" smd rect (at 3.6 -0.325) (locked) (size 1.75 0.45) (layers "F.Cu" "F.Paste" "F.Mask") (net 24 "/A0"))
  (pad "23" smd rect (at 3.6 -0.975) (locked) (size 1.75 0.45) (layers "F.Cu" "F.Paste" "F.Mask") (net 8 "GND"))
  (pad "24" smd rect (at 3.6 -1.625) (locked) (size 1.75 0.45) (layers "F.Cu" "F.Paste" "F.Mask") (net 25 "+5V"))
  (pad "25" smd rect (at 3.6 -2.275) (locked) (size 1.75 0.45) (layers "F.Cu" "F.Paste" "F.Mask") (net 26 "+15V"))
  (pad "26" smd rect (at 3.6 -2.925) (locked) (size 1.75 0.45) (layers "F.Cu" "F.Paste" "F.Mask") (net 62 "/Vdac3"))
  (pad "27" smd rect (at 3.6 -3.575) (locked) (size 1.75 0.45) (layers "F.Cu" "F.Paste" "F.Mask") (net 50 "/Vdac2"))
  (pad "28" smd rect (at 3.6 -4.225) (locked) (size 1.75 0.45) (layers "F.Cu" "F.Paste" "F.Mask") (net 29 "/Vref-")))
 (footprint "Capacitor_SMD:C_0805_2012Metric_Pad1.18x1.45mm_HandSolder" (layer "F.Cu") (at -8.5 50.5 -90)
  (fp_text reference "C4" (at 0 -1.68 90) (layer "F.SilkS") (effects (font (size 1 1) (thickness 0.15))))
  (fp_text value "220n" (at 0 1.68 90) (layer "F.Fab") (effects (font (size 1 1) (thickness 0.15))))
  (pad "1" smd roundrect (at -1.0375 0 270) (locked) (size 1.175 1.45) (layers "F.Cu" "F.Paste" "F.Mask") (roundrect_rratio 0.212766)
   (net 4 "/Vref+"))
  (pad "2" smd roundrect (at 1.0375 0 270) (locked) (size 1.175 1.45) (layers "F.Cu" "F.Paste" "F.Mask") (roundrect_rratio 0.212766)
   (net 8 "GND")))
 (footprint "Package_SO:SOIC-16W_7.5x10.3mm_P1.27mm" (layer "F.Cu") (at 0 51)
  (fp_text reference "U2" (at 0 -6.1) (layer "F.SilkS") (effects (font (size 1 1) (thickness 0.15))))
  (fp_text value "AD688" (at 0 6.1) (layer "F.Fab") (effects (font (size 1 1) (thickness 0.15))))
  (pad "1" smd roundrect (at -4.65 -4.445) (locked) (size 2.05 0.6) (layers "F.Cu" "F.Paste" "F.Mask") (roundrect_rratio 0.25)
   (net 35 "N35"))
  (pad "2" smd roundrect (at -4.65 -3.175) (locked) (size 2.05 0.6) (layers "F.Cu" "F.Paste" "F.Mask") (roundrect_rratio 0.25)
   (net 26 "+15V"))
  (pad "3" smd roundrect (at -4.65 -1.905) (locked) (size 2.05 0.6) (layers "F.Cu" "F.Paste" "F.Mask") (roundrect_rratio 0.25)
   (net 4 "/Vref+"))
  (pad "4" smd roundrect (at -4.65 -0.635) (locked) (size 2.05 0.6) (layers "F.Cu" "F.Paste" "F.Mask") (roundrect_rratio 0.25) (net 1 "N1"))
  (pad "5" smd roundrect (at -4.65 0.635) (locked) (size 2.05 0.6) (layers "F.Cu" "F.Paste" "F.Mask") (roundrect_rratio 0.25) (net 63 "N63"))
  (pad "6" smd roundrect (at -4.65 1.905) (locked) (size 2.05 0.6) (layers "F.Cu" "F.Paste" "F.Mask") (roundrect_rratio 0.25) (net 1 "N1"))
  (pad "7" smd roundrect (at -4.65 3.175) (locked) (size 2.05 0.6) (layers "F.Cu" "F.Paste" "F.Mask") (roundrect_rratio 0.25) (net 36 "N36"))
  (pad "8" smd roundrect (at -4.65 4.445) (locked) (size 2.05 0.6) (layers "F.Cu" "F.Paste" "F.Mask") (roundrect_rratio 0.25) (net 3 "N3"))
  (pad "9" smd roundrect (at 4.65 4.445) (locked) (size 2.05 0.6) (layers "F.Cu" "F.Paste" "F.Mask") (roundrect_rratio 0.25) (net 8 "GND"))
  (pad "10" smd roundrect (at 4.65 3.175) (locked) (size 2.05 0.6) (layers "F.Cu" "F.Paste" "F.Mask") (roundrect_rratio 0.25) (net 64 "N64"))
  (pad "11" smd roundrect (at 4.65 1.905) (locked) (size 2.05 0.6) (layers "F.Cu" "F.Paste" "F.Mask") (roundrect_rratio 0.25) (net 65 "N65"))
  (pad "12" smd roundrect (at 4.65 0.635) (locked) (size 2.05 0.6) (layers "F.Cu" "F.Paste" "F.Mask") (roundrect_rratio 0.25) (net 2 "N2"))
  (pad "13" smd roundrect (at 4.65 -0.635) (locked) (size 2.05 0.6) (layers "F.Cu" "F.Paste" "F.Mask") (roundrect_rratio 0.25) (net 3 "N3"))
  (pad "14" smd roundrect (at 4.65 -1.905) (locked) (size 2.05 0.6) (layers "F.Cu" "F.Paste" "F.Mask") (roundrect_rratio 0.25)
   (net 29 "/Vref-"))
  (pad "15" smd roundrect (at 4.65 -3.175) (locked) (size 2.05 0.6) (layers "F.Cu" "F.Paste" "F.Mask") (roundrect_rratio 0.25)
   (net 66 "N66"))
  (pad "16" smd roundrect (at 4.65 -4.445) (locked) (size 2.05 0.6) (layers "F.Cu" "F.Paste" "F.Mask") (roundrect_rratio 0.25)
   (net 7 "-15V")))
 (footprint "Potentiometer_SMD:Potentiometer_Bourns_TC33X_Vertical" (layer "F.Cu") (at -12.5 55 90)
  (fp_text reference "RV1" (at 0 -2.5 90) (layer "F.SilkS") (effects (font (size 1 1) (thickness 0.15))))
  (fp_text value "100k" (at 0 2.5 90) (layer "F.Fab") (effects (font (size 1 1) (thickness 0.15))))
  (pad "1" smd rect (at -1.8 -1 90) (locked) (size 1.2 1.2) (layers "F.Cu" "F.Paste" "F.Mask") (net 1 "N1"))
  (pad "2" smd rect (at 1.45 0 90) (locked) (size 1.5 1.6) (layers "F.Cu" "F.Paste" "F.Mask") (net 63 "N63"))
  (pad "3" smd rect (at -1.8 1 90) (locked) (size 1.2 1.2) (layers "F.Cu" "F.Paste" "F.Mask") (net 3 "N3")))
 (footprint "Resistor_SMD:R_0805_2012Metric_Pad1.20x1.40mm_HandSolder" (layer "F.Cu") (at 9 50 90)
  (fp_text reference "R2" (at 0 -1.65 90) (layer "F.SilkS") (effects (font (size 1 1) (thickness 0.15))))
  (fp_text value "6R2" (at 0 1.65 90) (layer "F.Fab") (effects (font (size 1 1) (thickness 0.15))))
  (pad "1" smd roundrect (at -1 0 90) (locked) (size 1.2 1.4) (layers "F.Cu" "F.Paste" "F.Mask") (roundrect_rratio 0.208333)
   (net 29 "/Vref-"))
  (pad "2" smd roundrect (at 1 0 90) (locked) (size 1.2 1.4) (layers "F.Cu" "F.Paste" "F.Mask") (roundrect_rratio 0.208333) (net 66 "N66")))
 (segment (start 35.6 38.9875) (end 39.4875 38.9875) (width 0.25) (layer "F.Cu") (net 8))
 (segment (start 39.5 54.0375) (end 35.6125 54.0375) (width 0.25) (layer "F.Cu") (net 8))
 (segment (start 24.5 54.0375) (end 25.1625 53.375) (width 0.25) (layer "F.Cu") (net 8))
 (segment (start 25.1625 38.3375) (end 28.4 38.3375) (width 0.25) (layer "F.Cu") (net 8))
 (segment (start 35.6125 54.0375) (end 35.6 54.025) (width 0.25) (layer "F.Cu") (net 8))
 (segment (start 11.5 48.9625) (end 11.425 48.9625) (width 0.25) (layer "F.Cu") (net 8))
 (segment (start 25.1625 53.375) (end 28.4 53.375) (width 0.25) (layer "F.Cu") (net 8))
 (segment (start 24.5 39) (end 25.1625 38.3375) (width 0.25) (layer "F.Cu") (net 8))
 (segment (start 39.4875 38.9875) (end 39.5 39) (width 0.25) (layer "F.Cu") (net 8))
 (segment (start 11.425 48.9625) (end 9 46.5375) (width 0.25) (layer "F.Cu") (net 8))
 (segment (start 38.7375 37.6875) (end 35.6 37.6875) (width 0.25) (layer "F.Cu") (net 26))
 (segment (start 38.7375 52.725) (end 39.5 51.9625) (width 0.25) (layer "F.Cu") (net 26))
 (segment (start -8.5 47.0375) (end -7.7125 47.825) (width 0.25) (layer "F.Cu") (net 26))
 (segment (start 35.6 52.725) (end 38.7375 52.725) (width 0.25) (layer "F.Cu") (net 26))
 (segment (start -7.7125 47.825) (end -4.65 47.825) (width 0.25) (layer "F.Cu") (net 26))
 (segment (start 39.5 36.925) (end 38.7375 37.6875) (width 0.25) (layer "F.Cu") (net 26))
 (segment (start 25.2625 52.725) (end 28.4 52.725) (width 0.25) (layer "F.Cu") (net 7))
 (segment (start 24.5 51.9625) (end 25.2625 52.725) (width 0.25) (layer "F.Cu") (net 7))
 (segment (start 9 44.4625) (end 6.7425 44.4625) (width 0.25) (layer "F.Cu") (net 7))
 (segment (start 24.5 36.925) (end 25.2625 37.6875) (width 0.25) (layer "F.Cu") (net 7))
 (segment (start 25.2625 37.6875) (end 28.4 37.6875) (width 0.25) (layer "F.Cu") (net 7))
 (segment (start 6.7425 44.4625) (end 4.65 46.555) (width 0.25) (layer "F.Cu") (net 7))
 (segment (start -8.2875 54.175) (end -8.5 53.9625) (width 0.25) (layer "F.Cu") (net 36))
 (segment (start -4.65 54.175) (end -8.2875 54.175) (width 0.25) (layer "F.Cu") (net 36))
 (segment (start -4.65 49.095) (end -8.1325 49.095) (width 0.2) (layer "F.Cu") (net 4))
 (segment (start -8.1325 49.095) (end -8.5 49.4625) (width 0.2) (layer "F.Cu") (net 4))
 (segment (start 9.0375 51.0375) (end 9 51) (width 0.2) (layer "F.Cu") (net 29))
 (segment (start 11.5 51.0375) (end 9.0375 51.0375) (width 0.2) (layer "F.Cu") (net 29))
 (segment (start 108.1375 35) (end 108.14 35.0025) (width 0.25) (layer "F.Cu") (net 25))
 (segment (start 104.115 33.73) (end 106.8675 33.73) (width 0.25) (layer "F.Cu") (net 25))
 (segment (start 104.115 36.27) (end 106.8725 36.27) (width 0.25) (layer "F.Cu") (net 25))
 (segment (start 104.115 35) (end 108.1375 35) (width 0.25) (layer "F.Cu") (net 25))
 (segment (start 106.8725 36.27) (end 108.14 35.0025) (width 0.25) (layer "F.Cu") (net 25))
 (segment (start 106.8675 33.73) (end 108.14 35.0025) (width 0.25) (layer "F.Cu") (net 25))
 (segment (start 104.115 45.69) (end 107.8675 45.69) (width 0.25) (layer "F.Cu") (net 25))
 (segment (start 107.8675 45.69) (end 108.14 45.9625) (width 0.25) (layer "F.Cu") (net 25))
 (segment (start 99.165 33.73) (end 100.87 33.73) (width 0.25) (layer "F.Cu") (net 30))
 (segment (start 100.87 33.73) (end 101.14 34) (width 0.25) (layer "F.Cu") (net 30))
 (segment (start 99.165 45.69) (end 99.165 46.96) (width 0.25) (layer "F.Cu") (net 30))
 (segment (start 100.83 45.69) (end 101.14 46) (width 0.25) (layer "F.Cu") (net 30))
 (segment (start 99.165 45.69) (end 100.83 45.69) (width 0.25) (layer "F.Cu") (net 30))
 (segment (start 99.165 35) (end 99.165 33.73) (width 0.25) (layer "F.Cu") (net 30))
 (via (at 101.14 34) (size 0.8) (drill 0.4) (layers "F.Cu" "B.Cu") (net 30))
 (via (at 101.14 46) (size 0.8) (drill 0.4) (layers "F.Cu" "B.Cu") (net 30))
 (segment (start 101.14 46) (end 101.14 34) (width 0.25) (layer "B.Cu") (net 30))
 (segment (start 101.14 46) (end 103.82 48.68) (width 0.25) (layer "B.Cu") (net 30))
 (segment (start 100.82 49.5) (end 99.165 49.5) (width 0.25) (layer "F.Cu") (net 32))
 (segment (start 99.165 38.81) (end 98.19 38.81) (width 0.25) (layer "F.Cu") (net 32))
 (segment (start 97.86498 39.13502) (end 97.86498 49.17498) (width 0.25) (layer "F.Cu") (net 32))
 (segment (start 98.19 38.81) (end 97.86498 39.13502) (width 0.25) (layer "F.Cu") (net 32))
 (segment (start 98.19 49.5) (end 99.165 49.5) (width 0.25) (layer "F.Cu") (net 32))
 (segment (start 99.165 50.77) (end 99.165 49.5) (width 0.25) (layer "F.Cu") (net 32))
 (segment (start 97.86498 49.17498) (end 98.19 49.5) (width 0.25) (layer "F.Cu") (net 32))
 (via (at 100.82 49.5) (size 0.8) (drill 0.4) (layers "F.Cu" "B.Cu") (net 32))
 (segment (start 102.82 51.5) (end 100.82 49.5) (width 0.25) (layer "B.Cu") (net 32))
 (segment (start -5.5 45.705) (end -5.5 43) (width 0.25) (layer "F.Cu") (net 35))
 (segment (start -4.65 46.555) (end -5.5 45.705) (width 0.25) (layer "F.Cu") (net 35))
 (segment (start 7.825 47.825) (end 4.65 47.825) (width 0.25) (layer "F.Cu") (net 66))
 (segment (start 9 49) (end 7.825 47.825) (width 0.25) (layer "F.Cu") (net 66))
 (segment (start -6.49002 52.45002) (end -5.675 51.635) (width 0.25) (layer "F.Cu") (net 63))
 (segment (start -11.40002 52.45002) (end -6.49002 52.45002) (width 0.25) (layer "F.Cu") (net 63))
 (segment (start -12.5 53.55) (end -11.40002 52.45002) (width 0.25) (layer "F.Cu") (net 63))
 (segment (start -5.675 51.635) (end -4.65 51.635) (width 0.25) (layer "F.Cu") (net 63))
 (segment (start 4.22322 50.365) (end 4.65 50.365) (width 0.25) (layer "F.Cu") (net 3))
 (segment (start -4.65 55.445) (end -0.85678 55.445) (width 0.25) (layer "F.Cu") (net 3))
 (segment (start -4.65 59.85) (end -4.65 55.445) (width 0.25) (layer "F.Cu") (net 3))
 (segment (start -6.15502 56.95002) (end -4.65 55.445) (width 0.25) (layer "F.Cu") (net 3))
 (segment (start -5.8 61) (end -4.65 59.85) (width 0.25) (layer "F.Cu") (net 3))
 (segment (start -11.34998 56.95002) (end -6.15502 56.95002) (width 0.25) (layer "F.Cu") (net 3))
 (segment (start -0.85678 55.445) (end 4.22322 50.365) (width 0.25) (layer "F.Cu") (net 3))
 (segment (start -11.5 56.8) (end -11.34998 56.95002) (width 0.25) (layer "F.Cu") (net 3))
 (segment (start -13.5 56.8) (end -11.3 59) (width 0.25) (layer "F.Cu") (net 1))
 (segment (start -11.3 59) (end -5.8 59) (width 0.25) (layer "F.Cu") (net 1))
 (segment (start -2.55 57.81) (end 3.625 51.635) (width 0.25) (layer "F.Cu") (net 2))
 (segment (start 3.625 51.635) (end 4.65 51.635) (width 0.25) (layer "F.Cu") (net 2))
 (segment (start -2.55 60) (end -2.55 57.81) (width 0.25) (layer "F.Cu") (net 2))
 (segment (start 104.115 38.81) (end 104.115 40.08) (width 0.25) (layer "F.Cu") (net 38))
 (segment (start 99.165 40.08) (end 104.115 40.08) (width 0.25) (layer "F.Cu") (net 38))
 (segment (start 99.165 37.54) (end 99.165 36.27) (width 0.25) (layer "F.Cu") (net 37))
 (segment (start 103.73822 48.23) (end 104.115 48.23) (width 0.25) (layer "F.Cu") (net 33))
 (segment (start 99.92822 52.04) (end 103.73822 48.23) (width 0.25) (layer "F.Cu") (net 33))
 (segment (start 99.165 52.04) (end 99.92822 52.04) (width 0.25) (layer "F.Cu") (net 33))
 (segment (start 104.115 50.77) (end 104.115 52.04) (width 0.25) (layer "F.Cu") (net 34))
 (segment (start 104.115 49.5) (end 104.115 50.77) (width 0.25) (layer "F.Cu") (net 34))
 (segment (start 100.14 48.23) (end 101.41 46.96) (width 0.25) (layer "F.Cu") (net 31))
 (segment (start 99.165 48.23) (end 100.14 48.23) (width 0.25) (layer "F.Cu") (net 31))
 (segment (start 101.41 46.96) (end 104.115 46.96) (width 0.25) (layer "F.Cu") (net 31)))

